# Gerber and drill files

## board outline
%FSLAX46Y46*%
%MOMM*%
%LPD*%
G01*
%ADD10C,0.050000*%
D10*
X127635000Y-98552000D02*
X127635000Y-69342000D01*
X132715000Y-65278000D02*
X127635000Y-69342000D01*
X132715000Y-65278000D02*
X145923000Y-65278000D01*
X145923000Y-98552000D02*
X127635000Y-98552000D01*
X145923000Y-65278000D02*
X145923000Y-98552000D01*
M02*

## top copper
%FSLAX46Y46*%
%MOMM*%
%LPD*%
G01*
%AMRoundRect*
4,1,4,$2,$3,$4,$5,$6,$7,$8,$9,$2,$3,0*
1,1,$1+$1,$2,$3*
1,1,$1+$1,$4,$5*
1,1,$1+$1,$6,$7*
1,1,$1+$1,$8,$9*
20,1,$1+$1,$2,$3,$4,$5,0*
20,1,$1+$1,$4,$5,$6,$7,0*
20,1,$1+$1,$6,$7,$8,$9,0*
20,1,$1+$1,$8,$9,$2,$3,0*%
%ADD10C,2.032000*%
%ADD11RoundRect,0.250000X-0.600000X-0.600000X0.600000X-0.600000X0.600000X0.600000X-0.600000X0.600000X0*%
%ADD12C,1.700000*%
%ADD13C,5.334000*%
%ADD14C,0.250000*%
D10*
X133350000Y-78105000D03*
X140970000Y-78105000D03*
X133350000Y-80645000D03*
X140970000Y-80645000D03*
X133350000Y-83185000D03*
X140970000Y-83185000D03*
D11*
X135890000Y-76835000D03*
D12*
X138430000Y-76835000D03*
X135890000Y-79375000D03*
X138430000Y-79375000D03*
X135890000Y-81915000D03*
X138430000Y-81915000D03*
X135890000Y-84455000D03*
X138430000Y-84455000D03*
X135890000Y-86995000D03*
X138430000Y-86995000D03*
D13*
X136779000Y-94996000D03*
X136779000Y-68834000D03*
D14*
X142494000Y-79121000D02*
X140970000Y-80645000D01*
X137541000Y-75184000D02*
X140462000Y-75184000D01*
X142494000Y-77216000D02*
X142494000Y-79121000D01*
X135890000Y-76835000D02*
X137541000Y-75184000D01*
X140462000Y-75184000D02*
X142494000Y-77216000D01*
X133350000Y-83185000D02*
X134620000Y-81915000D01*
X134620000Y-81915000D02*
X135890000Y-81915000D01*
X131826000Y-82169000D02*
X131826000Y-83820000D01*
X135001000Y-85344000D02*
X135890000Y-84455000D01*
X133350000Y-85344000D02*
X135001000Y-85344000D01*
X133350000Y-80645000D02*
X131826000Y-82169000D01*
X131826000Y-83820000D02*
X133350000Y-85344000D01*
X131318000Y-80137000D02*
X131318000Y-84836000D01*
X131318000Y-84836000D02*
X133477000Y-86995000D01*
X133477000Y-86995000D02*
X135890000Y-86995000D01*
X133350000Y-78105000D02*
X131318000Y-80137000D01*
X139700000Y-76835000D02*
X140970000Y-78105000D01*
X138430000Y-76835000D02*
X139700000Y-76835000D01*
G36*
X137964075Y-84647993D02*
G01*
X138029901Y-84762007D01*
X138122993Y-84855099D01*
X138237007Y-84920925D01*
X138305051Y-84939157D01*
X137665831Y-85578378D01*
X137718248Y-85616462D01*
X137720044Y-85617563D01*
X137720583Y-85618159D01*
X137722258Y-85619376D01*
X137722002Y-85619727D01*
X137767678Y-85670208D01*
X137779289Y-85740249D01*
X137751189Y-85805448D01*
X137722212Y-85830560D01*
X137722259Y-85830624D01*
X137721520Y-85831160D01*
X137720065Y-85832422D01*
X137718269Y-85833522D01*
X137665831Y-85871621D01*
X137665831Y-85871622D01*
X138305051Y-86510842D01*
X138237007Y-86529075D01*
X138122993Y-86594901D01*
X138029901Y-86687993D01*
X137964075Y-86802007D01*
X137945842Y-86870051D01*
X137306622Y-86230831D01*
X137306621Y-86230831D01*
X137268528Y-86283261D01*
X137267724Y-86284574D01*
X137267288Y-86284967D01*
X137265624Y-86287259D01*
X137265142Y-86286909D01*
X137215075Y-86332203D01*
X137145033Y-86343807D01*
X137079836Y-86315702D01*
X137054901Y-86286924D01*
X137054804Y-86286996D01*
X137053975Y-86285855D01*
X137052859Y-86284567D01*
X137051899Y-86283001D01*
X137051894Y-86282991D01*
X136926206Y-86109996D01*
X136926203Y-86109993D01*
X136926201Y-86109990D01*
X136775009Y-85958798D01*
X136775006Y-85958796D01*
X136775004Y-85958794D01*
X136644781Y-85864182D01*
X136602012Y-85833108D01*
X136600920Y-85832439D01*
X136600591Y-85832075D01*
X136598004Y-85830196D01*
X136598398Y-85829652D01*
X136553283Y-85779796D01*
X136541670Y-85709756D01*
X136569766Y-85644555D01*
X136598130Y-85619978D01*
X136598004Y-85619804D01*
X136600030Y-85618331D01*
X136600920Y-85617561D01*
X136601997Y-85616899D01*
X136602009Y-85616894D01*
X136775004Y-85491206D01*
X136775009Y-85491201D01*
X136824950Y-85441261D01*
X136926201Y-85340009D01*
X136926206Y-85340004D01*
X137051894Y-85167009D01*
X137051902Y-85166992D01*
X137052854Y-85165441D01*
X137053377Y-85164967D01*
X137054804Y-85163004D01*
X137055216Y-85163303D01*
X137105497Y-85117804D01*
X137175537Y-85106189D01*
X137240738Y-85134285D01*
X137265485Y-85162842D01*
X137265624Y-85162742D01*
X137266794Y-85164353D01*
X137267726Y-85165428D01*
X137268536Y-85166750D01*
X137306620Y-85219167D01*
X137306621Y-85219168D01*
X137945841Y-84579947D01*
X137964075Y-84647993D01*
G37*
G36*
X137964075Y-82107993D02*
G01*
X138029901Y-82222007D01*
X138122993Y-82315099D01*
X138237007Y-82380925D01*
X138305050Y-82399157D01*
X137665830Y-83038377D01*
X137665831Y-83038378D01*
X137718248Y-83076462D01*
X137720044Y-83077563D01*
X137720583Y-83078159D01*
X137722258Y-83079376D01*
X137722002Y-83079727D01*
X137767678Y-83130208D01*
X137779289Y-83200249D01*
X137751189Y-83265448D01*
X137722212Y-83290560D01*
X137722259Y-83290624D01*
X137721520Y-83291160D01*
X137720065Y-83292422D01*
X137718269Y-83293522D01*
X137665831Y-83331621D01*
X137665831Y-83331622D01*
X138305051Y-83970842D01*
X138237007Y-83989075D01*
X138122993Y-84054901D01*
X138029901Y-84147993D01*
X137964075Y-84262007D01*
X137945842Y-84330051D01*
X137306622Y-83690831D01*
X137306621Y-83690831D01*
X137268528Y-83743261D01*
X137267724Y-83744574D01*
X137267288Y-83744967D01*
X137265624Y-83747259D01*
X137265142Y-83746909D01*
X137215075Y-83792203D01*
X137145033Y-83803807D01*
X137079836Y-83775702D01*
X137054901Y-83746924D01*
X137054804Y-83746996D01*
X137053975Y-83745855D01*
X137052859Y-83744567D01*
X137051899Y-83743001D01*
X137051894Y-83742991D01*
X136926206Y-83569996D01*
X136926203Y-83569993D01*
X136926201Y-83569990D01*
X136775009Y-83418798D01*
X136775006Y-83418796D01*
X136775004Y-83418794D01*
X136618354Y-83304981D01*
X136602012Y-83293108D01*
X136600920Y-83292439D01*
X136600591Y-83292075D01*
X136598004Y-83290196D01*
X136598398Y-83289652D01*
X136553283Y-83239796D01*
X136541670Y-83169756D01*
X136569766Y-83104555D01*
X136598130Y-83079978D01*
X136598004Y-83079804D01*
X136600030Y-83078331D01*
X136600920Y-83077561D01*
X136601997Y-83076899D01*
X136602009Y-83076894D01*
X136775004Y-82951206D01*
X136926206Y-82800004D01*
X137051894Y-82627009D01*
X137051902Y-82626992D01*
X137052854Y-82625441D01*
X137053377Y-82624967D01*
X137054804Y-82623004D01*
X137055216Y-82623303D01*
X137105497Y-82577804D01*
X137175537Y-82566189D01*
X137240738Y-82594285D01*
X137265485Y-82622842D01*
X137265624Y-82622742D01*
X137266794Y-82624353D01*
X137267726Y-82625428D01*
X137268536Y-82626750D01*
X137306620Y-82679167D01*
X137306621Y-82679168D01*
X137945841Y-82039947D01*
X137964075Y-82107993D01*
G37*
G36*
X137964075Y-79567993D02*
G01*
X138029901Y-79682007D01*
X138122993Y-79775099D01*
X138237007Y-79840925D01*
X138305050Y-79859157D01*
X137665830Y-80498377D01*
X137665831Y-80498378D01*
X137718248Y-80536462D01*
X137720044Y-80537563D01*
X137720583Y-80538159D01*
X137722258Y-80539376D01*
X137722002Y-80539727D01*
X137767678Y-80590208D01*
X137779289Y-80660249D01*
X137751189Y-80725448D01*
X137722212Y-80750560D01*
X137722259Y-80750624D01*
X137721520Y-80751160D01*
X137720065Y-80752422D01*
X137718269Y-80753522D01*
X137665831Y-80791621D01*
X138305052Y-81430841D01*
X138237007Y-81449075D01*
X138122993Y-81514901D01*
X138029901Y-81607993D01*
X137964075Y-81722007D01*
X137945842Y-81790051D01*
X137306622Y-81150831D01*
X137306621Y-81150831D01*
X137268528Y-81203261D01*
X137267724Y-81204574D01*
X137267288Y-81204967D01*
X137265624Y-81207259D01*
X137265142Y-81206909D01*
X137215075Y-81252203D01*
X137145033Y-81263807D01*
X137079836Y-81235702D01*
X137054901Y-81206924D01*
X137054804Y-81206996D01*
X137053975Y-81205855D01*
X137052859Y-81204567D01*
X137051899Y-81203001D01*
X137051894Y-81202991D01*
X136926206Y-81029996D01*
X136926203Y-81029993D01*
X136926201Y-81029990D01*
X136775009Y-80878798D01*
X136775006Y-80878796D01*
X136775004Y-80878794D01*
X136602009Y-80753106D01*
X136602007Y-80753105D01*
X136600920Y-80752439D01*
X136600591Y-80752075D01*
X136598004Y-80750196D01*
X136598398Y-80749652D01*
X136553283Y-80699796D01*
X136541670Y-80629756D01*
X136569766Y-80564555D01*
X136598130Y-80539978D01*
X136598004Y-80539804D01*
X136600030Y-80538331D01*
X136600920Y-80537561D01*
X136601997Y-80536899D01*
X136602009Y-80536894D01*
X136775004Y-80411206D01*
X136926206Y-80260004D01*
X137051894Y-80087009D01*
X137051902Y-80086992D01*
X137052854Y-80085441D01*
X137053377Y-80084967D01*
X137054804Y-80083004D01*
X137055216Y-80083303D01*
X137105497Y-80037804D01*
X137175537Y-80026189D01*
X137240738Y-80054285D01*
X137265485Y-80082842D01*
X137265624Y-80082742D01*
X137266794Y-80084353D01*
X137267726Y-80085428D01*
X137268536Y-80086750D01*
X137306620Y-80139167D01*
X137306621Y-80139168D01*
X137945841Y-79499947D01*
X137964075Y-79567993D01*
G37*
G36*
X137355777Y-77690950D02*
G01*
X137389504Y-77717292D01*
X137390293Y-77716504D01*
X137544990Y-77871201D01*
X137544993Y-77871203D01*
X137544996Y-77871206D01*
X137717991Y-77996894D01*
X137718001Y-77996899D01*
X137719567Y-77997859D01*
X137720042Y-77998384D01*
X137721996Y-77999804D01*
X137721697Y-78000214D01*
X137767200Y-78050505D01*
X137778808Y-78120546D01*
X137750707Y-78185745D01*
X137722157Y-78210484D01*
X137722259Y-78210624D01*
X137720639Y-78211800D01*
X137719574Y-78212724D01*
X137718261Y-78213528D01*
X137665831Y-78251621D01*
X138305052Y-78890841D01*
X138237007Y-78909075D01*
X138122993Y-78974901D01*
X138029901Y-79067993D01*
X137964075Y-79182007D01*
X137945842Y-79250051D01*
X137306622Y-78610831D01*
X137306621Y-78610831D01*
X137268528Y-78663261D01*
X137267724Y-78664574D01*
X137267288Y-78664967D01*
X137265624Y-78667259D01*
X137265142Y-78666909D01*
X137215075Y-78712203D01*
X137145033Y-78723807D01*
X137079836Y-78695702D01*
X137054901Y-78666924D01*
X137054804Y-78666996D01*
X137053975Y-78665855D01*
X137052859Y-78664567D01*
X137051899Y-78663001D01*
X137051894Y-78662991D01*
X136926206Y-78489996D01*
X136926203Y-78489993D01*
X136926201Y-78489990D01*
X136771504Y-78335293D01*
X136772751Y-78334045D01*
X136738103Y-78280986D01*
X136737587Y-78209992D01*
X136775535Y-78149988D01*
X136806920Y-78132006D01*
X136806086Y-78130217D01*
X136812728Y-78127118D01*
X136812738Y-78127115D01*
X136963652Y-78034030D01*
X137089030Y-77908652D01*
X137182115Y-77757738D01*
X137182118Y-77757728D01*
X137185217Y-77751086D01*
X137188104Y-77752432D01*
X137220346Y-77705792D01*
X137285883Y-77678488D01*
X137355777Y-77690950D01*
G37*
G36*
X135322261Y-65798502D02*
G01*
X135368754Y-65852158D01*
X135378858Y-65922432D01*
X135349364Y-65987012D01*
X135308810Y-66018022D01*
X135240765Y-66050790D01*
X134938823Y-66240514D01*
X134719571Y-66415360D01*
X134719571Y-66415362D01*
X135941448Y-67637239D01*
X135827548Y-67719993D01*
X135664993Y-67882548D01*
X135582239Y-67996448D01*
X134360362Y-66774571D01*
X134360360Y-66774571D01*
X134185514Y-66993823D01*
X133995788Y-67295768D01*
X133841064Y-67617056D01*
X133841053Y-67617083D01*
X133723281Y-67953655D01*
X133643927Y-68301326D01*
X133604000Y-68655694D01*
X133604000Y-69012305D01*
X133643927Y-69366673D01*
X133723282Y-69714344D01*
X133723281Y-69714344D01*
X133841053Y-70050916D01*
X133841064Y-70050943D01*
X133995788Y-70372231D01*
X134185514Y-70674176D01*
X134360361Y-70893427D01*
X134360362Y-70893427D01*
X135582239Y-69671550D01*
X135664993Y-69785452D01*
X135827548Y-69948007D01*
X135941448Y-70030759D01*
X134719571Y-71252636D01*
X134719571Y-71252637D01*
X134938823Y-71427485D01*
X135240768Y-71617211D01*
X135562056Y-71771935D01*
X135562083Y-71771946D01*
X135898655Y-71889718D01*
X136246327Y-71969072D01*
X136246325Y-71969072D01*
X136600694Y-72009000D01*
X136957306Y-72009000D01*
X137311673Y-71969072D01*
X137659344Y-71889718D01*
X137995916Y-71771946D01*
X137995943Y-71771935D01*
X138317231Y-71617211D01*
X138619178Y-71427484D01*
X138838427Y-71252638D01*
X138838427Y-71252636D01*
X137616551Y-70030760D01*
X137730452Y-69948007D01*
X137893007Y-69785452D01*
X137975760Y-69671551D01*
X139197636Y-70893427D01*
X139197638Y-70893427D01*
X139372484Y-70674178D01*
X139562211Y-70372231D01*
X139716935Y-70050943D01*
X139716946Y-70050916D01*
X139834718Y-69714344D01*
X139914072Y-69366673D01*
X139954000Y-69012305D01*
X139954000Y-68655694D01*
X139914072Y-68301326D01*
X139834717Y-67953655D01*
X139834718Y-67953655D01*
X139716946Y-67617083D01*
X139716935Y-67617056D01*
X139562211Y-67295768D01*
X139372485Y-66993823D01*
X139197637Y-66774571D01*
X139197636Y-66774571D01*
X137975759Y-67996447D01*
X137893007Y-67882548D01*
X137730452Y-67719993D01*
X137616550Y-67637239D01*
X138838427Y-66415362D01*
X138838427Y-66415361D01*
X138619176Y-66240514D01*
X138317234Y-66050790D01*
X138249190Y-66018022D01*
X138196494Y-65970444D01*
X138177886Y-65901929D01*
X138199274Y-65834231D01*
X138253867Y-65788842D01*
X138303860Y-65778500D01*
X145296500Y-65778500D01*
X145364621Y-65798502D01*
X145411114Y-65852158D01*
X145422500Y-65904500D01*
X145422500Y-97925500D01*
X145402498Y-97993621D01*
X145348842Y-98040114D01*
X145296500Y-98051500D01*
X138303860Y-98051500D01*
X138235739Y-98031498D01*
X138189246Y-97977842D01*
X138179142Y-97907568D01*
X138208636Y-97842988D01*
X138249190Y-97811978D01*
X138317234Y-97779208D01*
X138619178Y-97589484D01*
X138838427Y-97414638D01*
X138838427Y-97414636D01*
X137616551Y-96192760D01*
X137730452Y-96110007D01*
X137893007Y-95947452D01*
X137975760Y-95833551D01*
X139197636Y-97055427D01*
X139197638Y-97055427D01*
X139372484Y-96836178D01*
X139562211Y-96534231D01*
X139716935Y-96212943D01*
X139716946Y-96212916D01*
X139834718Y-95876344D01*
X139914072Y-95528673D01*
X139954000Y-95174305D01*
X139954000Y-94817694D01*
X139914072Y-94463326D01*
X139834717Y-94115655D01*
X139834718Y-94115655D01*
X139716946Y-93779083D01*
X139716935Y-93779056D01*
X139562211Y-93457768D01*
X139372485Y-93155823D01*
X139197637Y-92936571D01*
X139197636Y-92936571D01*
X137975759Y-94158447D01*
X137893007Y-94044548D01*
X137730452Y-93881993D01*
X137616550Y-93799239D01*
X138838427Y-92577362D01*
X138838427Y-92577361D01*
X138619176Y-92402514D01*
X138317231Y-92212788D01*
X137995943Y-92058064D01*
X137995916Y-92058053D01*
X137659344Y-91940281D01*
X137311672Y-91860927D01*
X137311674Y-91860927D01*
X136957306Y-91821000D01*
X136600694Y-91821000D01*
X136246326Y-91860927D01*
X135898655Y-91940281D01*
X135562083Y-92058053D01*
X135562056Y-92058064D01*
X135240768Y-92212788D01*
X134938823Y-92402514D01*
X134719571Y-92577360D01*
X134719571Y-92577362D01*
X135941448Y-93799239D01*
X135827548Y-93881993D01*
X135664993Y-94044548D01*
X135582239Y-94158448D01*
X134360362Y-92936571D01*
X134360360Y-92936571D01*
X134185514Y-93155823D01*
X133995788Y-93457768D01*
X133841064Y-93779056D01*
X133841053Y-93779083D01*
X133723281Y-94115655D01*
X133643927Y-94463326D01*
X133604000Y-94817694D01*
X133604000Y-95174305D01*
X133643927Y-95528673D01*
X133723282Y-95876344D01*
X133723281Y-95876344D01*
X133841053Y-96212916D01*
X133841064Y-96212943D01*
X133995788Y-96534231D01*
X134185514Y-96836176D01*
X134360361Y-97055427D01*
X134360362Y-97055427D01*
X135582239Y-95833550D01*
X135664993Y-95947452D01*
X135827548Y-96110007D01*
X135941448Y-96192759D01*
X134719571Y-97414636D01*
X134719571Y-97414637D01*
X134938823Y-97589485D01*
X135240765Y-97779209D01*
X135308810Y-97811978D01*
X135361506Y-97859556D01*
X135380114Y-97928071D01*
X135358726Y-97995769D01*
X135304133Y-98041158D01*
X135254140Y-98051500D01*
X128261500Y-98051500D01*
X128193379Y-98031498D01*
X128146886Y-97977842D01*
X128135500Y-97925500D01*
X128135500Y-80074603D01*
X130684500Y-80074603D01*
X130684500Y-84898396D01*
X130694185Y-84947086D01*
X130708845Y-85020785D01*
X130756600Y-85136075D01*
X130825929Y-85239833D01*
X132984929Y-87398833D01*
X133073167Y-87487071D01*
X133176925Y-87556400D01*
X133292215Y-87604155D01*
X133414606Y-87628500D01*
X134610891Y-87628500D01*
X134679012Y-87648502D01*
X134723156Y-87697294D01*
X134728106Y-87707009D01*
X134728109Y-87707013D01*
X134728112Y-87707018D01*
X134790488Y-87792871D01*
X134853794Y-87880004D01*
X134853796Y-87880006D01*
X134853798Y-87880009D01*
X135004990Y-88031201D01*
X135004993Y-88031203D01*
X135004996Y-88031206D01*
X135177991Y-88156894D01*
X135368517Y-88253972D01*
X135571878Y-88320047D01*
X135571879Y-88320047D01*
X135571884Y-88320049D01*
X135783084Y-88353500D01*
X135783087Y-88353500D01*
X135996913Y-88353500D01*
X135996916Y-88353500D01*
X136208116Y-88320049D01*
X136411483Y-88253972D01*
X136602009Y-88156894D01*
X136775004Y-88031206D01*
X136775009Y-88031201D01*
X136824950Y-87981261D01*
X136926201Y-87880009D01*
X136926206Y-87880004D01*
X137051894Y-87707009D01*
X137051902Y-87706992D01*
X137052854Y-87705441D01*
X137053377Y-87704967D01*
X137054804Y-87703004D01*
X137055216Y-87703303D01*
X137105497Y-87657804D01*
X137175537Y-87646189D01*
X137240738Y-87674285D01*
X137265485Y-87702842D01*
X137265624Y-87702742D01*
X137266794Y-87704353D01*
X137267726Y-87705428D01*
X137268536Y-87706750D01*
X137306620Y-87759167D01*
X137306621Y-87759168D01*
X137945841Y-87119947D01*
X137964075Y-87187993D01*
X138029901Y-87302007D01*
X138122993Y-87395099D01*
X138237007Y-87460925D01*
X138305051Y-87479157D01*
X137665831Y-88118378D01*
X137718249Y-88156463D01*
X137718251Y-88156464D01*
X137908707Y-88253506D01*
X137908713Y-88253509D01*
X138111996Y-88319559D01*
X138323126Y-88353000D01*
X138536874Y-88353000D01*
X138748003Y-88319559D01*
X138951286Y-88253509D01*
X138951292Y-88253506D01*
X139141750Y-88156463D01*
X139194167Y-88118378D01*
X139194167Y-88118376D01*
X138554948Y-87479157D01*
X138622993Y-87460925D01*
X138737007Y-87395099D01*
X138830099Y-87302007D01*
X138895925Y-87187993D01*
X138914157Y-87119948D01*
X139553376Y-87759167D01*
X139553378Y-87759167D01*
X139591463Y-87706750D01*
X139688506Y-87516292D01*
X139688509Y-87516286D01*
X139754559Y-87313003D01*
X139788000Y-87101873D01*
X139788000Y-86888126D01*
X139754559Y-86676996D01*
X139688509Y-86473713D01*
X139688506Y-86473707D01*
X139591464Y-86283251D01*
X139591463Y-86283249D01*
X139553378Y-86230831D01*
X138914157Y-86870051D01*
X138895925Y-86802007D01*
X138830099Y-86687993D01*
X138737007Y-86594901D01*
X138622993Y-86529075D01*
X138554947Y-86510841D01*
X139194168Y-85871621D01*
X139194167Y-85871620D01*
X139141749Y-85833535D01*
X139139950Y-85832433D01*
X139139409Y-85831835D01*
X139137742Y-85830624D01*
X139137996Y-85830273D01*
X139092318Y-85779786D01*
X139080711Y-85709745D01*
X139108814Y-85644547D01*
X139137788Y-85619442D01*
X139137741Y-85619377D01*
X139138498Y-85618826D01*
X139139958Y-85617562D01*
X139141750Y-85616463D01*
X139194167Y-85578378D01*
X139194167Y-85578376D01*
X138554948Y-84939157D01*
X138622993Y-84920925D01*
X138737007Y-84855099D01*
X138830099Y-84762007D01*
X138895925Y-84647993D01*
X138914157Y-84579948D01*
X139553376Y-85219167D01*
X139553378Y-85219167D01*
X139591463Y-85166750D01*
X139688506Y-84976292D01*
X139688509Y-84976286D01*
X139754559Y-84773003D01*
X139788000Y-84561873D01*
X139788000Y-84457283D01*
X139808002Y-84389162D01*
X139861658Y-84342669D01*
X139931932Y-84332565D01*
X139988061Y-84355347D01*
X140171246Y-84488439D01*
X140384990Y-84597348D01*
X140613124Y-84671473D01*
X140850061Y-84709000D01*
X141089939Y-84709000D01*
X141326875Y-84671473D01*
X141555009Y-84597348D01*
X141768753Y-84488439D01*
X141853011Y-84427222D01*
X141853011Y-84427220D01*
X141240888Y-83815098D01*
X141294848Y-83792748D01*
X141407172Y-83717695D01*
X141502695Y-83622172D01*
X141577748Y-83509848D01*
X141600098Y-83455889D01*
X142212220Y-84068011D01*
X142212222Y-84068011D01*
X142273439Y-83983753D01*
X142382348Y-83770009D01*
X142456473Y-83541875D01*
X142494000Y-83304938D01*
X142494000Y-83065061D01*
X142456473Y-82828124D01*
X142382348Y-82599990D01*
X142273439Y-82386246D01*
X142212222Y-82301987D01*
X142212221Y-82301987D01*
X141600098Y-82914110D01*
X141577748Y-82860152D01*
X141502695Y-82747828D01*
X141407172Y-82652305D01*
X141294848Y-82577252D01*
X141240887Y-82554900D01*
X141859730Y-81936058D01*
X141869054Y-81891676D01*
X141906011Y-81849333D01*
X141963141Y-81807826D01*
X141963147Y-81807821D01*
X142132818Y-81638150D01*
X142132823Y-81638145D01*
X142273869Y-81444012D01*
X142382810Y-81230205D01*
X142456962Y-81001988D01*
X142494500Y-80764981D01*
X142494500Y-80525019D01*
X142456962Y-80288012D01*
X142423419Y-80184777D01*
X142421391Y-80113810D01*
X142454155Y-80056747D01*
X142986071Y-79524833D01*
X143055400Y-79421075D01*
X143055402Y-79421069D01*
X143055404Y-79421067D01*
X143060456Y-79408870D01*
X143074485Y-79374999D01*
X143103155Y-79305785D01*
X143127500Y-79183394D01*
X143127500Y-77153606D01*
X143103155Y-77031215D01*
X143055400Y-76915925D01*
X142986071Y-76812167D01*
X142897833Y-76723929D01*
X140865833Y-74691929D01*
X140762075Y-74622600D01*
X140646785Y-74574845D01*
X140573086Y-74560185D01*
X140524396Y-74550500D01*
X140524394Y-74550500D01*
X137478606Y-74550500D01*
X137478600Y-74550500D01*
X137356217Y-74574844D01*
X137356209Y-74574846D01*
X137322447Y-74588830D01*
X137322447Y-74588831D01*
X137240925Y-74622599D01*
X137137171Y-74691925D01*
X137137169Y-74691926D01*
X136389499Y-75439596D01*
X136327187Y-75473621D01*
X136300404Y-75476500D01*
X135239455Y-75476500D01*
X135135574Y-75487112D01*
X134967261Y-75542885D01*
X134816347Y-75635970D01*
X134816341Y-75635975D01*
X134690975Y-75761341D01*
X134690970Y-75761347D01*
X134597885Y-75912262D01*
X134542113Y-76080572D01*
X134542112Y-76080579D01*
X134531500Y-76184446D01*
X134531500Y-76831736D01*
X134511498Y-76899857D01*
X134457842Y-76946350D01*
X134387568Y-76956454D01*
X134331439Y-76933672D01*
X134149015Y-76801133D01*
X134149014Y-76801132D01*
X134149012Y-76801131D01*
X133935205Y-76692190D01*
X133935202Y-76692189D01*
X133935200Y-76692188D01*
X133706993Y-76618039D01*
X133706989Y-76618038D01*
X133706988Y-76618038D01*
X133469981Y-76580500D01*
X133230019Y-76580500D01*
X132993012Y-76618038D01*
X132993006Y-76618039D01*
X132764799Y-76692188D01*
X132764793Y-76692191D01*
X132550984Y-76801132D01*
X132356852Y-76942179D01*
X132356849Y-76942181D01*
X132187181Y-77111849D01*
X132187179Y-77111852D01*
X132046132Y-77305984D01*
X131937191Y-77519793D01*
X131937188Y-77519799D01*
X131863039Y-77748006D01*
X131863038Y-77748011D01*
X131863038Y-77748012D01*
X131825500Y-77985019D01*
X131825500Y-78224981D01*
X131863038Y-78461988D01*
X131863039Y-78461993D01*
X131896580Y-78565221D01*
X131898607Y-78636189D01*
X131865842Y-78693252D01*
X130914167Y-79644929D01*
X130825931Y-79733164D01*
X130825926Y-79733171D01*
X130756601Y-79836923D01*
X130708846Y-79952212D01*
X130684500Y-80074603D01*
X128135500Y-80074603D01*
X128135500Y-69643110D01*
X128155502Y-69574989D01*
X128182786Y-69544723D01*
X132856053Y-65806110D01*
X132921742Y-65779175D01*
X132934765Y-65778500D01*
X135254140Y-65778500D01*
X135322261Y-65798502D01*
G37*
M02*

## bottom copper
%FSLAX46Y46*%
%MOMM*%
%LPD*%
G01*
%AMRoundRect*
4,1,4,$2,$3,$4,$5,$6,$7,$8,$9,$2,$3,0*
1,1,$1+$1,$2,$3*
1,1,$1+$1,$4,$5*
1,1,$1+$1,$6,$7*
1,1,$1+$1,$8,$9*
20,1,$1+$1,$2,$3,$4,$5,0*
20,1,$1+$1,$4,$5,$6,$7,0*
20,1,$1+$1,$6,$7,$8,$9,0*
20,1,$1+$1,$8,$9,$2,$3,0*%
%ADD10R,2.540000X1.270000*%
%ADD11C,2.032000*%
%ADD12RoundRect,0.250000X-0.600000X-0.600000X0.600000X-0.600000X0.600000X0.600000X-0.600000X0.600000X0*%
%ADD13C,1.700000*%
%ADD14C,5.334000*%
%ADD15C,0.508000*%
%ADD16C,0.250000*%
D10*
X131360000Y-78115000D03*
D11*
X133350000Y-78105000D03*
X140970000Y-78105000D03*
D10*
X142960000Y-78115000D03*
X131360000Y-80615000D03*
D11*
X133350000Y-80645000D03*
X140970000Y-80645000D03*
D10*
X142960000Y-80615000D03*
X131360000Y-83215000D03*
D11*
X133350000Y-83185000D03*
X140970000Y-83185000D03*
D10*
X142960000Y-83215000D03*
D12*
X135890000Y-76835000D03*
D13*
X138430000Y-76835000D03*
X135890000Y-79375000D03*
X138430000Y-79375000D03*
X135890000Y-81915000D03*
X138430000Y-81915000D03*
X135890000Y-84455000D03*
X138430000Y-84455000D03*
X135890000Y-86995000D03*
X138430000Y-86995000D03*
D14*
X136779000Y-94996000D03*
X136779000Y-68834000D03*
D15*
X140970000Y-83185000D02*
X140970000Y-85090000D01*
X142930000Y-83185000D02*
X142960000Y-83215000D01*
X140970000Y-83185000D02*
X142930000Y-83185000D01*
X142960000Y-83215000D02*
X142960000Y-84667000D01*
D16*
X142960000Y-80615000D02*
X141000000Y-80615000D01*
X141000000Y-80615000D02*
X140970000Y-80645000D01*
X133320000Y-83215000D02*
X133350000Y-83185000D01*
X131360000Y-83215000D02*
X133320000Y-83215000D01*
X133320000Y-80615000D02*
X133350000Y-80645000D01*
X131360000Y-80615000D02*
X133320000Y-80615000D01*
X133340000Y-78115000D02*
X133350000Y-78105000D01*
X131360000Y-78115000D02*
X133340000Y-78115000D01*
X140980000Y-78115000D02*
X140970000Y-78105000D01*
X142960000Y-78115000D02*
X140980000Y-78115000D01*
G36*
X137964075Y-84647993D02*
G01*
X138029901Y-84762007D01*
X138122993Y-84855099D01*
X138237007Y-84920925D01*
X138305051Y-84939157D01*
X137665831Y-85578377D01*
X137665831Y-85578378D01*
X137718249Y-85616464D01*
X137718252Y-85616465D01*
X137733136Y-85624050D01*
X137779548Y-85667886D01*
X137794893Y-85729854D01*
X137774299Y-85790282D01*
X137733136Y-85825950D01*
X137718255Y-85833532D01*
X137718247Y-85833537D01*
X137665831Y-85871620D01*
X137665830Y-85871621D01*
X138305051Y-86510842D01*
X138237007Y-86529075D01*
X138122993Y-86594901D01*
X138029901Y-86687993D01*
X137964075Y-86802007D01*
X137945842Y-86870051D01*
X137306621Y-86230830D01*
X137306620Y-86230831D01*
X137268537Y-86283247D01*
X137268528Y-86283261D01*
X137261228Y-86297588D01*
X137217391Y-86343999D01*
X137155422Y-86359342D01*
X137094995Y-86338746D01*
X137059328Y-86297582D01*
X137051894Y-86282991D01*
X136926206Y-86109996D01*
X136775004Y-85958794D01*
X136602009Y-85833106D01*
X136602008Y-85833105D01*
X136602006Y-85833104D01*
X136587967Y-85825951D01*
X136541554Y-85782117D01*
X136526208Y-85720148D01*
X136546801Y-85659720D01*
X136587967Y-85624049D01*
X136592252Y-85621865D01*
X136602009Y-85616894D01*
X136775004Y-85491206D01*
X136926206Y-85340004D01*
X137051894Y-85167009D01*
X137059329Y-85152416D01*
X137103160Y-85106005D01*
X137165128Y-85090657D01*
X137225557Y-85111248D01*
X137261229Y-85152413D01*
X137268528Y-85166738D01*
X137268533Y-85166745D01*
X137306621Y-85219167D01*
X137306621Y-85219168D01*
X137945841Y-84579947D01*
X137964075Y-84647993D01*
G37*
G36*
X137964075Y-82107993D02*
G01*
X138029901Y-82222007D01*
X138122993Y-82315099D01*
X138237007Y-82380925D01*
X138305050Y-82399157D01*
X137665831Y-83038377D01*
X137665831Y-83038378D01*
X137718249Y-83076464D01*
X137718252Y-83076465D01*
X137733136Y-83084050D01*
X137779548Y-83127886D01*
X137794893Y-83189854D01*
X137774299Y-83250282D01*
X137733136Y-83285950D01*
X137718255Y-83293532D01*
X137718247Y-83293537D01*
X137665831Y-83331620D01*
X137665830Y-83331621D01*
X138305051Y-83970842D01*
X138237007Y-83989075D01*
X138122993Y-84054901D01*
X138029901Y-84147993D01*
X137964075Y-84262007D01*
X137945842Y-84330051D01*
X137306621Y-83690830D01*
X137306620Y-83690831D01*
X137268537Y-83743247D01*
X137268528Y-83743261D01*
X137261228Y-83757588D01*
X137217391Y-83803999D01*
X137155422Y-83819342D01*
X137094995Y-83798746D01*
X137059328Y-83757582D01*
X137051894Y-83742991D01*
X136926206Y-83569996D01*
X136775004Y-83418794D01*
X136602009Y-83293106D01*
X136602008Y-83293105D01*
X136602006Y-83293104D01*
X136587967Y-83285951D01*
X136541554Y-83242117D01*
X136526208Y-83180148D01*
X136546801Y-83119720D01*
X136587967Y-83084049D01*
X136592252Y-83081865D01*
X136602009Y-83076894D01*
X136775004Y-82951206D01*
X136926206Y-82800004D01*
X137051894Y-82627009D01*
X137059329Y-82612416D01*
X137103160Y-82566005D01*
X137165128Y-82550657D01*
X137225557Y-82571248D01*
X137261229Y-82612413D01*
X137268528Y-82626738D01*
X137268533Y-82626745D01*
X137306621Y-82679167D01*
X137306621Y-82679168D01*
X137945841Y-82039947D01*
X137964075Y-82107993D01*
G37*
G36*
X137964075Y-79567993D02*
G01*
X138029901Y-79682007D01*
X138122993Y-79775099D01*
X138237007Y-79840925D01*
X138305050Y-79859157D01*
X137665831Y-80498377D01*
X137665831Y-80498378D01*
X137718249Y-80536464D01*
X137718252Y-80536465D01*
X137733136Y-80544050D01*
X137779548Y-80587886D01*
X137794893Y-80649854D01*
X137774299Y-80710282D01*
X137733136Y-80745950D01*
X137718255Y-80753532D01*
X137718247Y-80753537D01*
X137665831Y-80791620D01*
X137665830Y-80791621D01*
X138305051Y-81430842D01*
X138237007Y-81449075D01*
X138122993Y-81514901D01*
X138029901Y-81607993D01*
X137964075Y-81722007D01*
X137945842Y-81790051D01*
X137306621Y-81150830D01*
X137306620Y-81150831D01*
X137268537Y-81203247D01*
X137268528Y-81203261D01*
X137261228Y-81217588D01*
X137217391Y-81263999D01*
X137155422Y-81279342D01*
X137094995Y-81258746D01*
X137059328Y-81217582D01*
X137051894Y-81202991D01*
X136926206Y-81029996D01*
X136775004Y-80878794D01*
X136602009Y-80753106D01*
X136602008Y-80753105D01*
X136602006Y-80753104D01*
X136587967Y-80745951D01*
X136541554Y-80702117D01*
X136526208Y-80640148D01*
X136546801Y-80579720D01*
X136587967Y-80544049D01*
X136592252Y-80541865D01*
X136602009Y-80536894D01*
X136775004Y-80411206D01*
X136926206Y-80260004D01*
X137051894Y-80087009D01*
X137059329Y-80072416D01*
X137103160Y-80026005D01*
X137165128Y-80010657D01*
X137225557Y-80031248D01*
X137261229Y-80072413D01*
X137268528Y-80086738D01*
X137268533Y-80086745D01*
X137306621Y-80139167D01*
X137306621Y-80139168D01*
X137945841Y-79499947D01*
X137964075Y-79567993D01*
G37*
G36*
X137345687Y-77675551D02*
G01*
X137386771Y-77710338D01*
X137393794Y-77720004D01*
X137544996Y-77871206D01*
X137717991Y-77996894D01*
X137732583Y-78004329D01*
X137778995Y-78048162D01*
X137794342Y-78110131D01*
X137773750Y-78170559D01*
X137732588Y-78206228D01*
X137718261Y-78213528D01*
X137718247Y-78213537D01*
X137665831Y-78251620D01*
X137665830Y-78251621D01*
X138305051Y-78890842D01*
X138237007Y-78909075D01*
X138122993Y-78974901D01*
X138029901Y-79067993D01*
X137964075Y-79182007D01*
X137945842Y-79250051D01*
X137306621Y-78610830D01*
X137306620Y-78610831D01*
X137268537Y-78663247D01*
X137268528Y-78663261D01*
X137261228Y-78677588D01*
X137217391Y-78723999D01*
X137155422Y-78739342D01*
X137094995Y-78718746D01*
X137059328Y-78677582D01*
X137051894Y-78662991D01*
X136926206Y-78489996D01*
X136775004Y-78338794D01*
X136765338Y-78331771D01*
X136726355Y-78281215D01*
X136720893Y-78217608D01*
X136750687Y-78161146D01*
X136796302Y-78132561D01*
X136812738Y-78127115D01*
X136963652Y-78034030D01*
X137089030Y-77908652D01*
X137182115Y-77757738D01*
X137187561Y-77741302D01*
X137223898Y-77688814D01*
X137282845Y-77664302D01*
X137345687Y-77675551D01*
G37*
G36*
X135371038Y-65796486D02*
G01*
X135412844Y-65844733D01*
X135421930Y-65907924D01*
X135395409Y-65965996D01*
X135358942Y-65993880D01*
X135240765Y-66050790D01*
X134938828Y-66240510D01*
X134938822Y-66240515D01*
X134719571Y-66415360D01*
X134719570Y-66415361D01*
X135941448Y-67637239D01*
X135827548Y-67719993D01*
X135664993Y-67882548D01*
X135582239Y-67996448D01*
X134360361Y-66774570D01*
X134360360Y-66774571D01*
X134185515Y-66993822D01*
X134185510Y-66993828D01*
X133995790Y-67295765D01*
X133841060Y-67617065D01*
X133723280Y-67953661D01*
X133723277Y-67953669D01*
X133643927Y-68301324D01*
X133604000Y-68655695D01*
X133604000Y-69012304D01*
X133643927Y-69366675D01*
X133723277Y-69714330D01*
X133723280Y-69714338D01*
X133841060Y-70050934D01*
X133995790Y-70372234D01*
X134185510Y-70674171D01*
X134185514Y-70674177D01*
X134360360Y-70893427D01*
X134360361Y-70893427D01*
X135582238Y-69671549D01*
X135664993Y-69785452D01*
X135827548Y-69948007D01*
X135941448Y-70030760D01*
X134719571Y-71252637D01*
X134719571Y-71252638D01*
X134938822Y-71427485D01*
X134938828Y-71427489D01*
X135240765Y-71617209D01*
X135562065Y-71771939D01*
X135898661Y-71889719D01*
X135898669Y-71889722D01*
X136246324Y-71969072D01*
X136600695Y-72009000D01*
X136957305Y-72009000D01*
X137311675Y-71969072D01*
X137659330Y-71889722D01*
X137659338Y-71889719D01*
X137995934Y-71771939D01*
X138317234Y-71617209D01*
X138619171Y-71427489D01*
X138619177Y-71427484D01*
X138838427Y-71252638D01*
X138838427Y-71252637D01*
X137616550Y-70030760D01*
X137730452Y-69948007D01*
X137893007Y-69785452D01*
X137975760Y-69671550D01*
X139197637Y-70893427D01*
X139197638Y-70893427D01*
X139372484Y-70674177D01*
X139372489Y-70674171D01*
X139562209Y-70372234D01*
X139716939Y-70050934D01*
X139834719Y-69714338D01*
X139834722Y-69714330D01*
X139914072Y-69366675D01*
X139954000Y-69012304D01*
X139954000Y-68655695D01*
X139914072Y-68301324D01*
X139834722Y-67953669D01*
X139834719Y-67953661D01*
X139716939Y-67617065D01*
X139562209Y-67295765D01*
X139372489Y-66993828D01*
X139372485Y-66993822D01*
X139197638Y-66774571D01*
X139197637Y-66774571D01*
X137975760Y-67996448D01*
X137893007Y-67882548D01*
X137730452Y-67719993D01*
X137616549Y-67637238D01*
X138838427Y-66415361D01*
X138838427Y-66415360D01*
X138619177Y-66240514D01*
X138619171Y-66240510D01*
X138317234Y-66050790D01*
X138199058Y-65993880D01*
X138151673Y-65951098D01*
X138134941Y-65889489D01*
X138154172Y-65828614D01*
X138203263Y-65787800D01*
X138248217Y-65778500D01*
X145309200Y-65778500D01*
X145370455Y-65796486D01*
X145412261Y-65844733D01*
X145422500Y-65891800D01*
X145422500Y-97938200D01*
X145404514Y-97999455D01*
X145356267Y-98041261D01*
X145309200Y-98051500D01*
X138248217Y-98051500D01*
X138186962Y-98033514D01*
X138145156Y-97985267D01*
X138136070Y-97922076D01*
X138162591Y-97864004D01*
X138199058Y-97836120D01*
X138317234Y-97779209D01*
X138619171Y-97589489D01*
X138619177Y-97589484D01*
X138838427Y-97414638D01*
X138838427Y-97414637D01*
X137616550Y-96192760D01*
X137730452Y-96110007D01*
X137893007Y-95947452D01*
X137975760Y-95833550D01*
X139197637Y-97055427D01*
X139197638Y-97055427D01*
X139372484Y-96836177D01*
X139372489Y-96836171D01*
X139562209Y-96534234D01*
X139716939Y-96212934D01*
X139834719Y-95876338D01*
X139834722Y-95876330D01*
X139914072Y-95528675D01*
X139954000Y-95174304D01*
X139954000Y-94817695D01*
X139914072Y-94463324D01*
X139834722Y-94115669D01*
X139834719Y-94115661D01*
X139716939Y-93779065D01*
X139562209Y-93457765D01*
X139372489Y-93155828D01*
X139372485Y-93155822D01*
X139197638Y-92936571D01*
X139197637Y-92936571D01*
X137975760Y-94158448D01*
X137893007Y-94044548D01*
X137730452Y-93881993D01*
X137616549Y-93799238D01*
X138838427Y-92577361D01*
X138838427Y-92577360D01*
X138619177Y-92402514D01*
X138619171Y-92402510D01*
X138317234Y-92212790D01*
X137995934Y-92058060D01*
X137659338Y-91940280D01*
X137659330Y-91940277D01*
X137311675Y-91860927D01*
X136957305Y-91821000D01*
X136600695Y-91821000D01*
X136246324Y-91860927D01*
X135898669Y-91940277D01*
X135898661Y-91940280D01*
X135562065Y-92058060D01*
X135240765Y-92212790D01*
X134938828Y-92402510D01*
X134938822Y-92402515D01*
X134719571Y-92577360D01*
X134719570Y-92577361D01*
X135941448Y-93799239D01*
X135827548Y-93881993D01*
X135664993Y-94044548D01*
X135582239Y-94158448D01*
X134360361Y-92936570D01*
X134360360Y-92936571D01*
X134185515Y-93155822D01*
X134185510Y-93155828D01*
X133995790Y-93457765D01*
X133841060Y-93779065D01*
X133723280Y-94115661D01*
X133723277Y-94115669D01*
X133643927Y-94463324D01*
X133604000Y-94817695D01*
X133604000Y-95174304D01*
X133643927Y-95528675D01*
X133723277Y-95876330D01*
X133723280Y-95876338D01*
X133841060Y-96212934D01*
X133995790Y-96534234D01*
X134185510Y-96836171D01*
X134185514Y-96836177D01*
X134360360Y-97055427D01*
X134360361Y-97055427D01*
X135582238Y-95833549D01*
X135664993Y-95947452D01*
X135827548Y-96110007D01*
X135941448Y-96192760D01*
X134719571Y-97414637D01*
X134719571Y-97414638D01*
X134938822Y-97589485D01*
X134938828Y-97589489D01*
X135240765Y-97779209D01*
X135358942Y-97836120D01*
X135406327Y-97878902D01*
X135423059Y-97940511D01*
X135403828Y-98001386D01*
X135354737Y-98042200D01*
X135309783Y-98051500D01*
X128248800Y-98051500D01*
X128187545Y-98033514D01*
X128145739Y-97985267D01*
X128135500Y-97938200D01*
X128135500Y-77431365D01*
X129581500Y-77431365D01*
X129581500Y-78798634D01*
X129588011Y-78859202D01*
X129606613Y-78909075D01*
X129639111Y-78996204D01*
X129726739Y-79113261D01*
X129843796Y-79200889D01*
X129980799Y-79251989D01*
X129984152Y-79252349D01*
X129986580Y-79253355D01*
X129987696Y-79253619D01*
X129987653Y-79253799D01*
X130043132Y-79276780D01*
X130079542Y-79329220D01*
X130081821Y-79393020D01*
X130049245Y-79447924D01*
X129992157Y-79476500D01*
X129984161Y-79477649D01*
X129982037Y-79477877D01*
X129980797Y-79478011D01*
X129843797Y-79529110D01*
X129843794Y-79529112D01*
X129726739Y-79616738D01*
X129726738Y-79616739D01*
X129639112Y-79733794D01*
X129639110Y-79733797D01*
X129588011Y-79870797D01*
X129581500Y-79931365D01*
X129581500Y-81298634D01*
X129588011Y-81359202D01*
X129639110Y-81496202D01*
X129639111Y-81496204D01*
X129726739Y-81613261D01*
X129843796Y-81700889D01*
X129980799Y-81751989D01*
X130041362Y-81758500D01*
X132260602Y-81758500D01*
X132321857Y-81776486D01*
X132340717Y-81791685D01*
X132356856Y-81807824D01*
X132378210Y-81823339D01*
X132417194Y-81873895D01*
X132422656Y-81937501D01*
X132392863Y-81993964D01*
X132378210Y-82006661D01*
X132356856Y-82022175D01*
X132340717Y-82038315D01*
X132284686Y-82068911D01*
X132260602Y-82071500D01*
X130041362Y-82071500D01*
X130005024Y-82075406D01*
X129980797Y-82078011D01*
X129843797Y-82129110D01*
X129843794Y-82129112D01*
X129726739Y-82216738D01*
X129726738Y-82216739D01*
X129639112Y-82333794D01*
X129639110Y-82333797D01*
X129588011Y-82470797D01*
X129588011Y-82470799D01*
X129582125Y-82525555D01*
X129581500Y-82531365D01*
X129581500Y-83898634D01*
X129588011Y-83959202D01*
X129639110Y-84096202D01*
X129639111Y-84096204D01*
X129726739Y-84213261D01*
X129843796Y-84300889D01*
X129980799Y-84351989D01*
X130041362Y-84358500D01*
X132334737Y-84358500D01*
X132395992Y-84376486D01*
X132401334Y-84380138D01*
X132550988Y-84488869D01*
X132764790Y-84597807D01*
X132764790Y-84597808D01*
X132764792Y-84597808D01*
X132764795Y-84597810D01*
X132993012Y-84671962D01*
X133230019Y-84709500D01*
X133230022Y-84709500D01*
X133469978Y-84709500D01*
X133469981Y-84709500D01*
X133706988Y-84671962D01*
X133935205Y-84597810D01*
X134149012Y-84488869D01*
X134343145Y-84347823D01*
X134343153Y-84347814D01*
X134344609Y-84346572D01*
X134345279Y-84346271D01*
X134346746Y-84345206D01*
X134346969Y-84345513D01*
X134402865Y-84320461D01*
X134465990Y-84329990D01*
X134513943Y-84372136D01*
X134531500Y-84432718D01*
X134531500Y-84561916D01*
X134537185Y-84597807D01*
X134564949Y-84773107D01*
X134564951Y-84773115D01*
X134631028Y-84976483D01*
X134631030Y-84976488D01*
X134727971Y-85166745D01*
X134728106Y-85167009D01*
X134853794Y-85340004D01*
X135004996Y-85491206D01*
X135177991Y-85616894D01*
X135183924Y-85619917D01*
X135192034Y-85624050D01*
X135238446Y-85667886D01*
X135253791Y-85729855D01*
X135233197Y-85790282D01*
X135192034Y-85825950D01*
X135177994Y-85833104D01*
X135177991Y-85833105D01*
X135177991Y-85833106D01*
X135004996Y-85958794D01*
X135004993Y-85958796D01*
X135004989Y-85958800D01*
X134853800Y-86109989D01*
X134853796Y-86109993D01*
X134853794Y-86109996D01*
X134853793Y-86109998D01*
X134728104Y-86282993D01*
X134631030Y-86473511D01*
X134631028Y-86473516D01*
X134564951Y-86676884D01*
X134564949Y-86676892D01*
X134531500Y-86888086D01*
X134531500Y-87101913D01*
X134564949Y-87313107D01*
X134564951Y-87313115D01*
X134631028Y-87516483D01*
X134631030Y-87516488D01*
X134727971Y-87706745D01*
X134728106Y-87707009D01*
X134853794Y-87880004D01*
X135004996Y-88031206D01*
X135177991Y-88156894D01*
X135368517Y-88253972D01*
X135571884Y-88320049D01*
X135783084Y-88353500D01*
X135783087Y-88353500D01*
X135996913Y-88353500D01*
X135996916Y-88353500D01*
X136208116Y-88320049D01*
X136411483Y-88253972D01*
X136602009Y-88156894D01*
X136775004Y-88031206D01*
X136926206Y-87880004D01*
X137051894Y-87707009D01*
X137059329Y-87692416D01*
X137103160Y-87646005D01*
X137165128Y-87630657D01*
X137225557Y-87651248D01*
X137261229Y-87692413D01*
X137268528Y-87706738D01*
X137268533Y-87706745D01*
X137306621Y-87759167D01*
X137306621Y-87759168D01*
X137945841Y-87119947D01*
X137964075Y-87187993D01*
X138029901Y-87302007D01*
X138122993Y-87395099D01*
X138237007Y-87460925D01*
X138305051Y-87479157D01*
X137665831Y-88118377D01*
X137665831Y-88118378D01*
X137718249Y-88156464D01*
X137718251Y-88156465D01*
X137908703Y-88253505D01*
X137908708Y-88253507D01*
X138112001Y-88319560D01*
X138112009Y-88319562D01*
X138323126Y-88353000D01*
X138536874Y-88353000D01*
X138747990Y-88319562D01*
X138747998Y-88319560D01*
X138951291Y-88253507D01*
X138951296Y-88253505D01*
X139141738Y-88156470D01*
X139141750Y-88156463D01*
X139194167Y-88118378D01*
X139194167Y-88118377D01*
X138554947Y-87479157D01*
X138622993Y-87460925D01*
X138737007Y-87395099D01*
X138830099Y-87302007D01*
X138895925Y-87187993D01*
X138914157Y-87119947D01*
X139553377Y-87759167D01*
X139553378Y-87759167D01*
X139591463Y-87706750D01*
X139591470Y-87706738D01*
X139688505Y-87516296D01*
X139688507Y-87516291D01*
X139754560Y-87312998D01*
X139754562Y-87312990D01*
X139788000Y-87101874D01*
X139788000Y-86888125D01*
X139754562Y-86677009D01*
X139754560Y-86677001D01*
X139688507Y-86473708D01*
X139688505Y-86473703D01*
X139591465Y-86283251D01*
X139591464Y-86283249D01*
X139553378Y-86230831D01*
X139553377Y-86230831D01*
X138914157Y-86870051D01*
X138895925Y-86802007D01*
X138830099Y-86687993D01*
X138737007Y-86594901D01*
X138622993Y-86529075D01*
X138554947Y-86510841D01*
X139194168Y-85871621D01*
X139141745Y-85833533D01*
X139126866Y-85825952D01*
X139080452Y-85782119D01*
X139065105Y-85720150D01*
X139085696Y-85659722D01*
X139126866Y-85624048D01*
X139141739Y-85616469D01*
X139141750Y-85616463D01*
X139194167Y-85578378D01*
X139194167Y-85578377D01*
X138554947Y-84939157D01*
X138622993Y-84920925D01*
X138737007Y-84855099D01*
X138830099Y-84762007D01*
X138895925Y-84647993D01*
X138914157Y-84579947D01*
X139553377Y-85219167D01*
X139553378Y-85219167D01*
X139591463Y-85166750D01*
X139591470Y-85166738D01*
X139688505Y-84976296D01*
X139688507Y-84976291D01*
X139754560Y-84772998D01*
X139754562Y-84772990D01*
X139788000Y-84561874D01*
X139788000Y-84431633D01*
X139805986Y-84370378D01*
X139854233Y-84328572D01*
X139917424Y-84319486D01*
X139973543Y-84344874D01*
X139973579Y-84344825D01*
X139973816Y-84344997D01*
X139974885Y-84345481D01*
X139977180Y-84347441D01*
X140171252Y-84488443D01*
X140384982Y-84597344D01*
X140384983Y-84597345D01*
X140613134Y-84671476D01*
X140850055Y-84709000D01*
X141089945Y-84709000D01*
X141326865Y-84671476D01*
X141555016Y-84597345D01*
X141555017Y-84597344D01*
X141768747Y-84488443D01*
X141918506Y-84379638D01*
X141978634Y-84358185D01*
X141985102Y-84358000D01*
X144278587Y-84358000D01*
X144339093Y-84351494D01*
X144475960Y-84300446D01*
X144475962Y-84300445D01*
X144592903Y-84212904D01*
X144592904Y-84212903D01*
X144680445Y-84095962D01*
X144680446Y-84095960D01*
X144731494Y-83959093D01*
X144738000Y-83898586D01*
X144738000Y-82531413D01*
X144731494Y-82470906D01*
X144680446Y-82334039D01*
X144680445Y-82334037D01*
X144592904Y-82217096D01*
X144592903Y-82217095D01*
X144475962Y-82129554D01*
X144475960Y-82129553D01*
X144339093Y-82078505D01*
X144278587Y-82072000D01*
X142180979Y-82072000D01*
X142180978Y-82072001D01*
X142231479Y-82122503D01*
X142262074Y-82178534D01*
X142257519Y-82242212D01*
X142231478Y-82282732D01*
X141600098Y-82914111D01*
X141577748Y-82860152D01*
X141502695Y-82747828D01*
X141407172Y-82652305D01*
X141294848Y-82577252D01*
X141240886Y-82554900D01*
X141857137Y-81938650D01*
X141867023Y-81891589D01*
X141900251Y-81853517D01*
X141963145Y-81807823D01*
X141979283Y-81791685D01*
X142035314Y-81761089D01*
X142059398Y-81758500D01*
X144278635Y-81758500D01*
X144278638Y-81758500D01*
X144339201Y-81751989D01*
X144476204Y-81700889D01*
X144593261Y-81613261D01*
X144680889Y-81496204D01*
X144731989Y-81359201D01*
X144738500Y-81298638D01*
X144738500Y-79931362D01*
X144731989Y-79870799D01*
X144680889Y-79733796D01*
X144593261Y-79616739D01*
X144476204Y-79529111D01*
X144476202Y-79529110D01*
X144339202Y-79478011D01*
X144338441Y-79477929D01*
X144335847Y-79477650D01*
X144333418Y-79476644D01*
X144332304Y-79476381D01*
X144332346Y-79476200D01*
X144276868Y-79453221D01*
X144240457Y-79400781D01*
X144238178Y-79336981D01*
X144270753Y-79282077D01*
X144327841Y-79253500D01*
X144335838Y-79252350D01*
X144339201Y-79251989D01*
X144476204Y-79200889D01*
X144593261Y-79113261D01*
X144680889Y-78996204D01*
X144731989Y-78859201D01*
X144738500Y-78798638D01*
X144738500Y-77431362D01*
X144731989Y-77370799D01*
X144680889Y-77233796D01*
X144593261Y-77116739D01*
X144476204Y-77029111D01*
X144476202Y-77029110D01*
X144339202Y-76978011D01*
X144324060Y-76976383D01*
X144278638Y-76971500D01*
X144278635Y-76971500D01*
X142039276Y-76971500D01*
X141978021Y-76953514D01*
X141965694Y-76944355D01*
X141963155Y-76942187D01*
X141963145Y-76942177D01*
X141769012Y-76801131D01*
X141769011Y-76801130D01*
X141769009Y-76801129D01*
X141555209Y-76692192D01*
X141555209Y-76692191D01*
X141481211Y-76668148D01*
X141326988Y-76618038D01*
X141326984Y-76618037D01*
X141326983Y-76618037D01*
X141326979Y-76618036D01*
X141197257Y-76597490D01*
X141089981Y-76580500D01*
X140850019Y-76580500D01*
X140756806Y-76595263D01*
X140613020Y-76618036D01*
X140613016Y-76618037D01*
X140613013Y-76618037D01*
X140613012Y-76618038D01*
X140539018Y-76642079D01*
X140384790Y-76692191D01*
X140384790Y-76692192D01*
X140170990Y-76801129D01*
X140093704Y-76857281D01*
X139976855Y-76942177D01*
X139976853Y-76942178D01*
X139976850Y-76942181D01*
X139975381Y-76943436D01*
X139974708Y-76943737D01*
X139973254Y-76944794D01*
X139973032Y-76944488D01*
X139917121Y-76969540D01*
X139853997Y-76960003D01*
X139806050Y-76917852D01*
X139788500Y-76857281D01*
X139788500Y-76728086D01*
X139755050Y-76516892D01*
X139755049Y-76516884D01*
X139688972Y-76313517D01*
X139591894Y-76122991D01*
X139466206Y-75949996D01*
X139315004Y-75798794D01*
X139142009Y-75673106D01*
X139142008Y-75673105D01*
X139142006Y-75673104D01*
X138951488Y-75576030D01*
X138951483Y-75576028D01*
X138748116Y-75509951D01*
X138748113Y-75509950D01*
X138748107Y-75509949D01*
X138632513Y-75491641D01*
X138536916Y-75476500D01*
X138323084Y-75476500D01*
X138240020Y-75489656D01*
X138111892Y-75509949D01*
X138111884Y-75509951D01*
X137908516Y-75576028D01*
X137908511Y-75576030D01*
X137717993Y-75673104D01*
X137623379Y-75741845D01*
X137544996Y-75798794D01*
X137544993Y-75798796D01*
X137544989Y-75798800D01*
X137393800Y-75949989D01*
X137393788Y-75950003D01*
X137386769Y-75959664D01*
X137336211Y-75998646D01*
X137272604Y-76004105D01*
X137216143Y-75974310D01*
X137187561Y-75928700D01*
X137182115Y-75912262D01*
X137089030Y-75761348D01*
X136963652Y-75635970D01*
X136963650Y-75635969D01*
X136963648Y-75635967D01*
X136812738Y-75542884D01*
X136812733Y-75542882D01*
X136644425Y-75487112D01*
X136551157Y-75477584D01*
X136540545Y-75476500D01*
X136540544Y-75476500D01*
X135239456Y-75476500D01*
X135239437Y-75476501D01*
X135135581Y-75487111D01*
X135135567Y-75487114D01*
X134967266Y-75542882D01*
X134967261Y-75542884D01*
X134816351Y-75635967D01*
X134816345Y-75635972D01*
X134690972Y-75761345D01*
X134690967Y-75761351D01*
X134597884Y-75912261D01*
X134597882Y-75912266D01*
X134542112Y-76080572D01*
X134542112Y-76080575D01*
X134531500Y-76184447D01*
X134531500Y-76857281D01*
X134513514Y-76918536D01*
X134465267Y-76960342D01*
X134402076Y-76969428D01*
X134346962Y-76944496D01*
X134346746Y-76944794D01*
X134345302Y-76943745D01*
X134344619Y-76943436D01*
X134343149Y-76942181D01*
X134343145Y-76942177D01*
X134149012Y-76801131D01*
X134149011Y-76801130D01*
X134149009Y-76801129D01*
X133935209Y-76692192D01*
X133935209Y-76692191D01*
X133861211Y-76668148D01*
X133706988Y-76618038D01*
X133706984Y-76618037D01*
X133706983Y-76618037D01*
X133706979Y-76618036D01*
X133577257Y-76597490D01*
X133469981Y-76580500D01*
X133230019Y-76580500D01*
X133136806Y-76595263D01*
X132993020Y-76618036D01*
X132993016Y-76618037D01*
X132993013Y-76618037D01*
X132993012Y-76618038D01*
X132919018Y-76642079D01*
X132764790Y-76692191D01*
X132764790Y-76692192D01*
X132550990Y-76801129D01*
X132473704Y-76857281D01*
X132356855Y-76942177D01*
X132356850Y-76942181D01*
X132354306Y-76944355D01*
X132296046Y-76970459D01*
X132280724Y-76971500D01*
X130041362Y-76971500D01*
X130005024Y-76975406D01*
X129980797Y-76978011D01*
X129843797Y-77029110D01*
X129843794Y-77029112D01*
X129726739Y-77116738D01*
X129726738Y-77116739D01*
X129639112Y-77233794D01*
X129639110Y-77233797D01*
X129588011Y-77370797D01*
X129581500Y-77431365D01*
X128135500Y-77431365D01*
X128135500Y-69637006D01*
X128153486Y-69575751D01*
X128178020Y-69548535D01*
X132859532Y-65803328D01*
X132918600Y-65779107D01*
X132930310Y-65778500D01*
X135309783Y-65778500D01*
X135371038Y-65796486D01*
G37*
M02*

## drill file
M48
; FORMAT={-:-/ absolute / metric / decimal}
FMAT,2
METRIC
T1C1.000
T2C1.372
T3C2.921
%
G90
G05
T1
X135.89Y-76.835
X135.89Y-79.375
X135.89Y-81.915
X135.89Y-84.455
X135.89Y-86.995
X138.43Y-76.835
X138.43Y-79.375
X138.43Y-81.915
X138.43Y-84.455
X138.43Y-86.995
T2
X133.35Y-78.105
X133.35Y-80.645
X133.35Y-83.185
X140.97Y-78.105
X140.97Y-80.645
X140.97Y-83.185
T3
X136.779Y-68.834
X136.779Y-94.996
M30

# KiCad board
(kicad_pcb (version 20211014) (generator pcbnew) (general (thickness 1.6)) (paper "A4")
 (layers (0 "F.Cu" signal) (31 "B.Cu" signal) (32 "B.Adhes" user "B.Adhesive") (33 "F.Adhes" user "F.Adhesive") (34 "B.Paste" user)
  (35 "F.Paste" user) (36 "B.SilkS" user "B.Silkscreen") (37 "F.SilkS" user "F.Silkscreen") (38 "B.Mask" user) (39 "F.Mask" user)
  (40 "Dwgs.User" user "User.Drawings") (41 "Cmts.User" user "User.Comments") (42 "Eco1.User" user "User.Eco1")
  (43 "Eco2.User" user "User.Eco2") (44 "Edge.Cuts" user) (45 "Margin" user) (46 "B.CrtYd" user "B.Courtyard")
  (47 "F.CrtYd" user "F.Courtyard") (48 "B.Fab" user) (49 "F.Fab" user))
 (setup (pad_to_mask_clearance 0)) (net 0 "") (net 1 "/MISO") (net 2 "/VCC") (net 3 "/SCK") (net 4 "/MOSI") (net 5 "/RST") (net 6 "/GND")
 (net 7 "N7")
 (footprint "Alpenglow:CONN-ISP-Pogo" (layer "F.Cu") (at 137.16 81.915)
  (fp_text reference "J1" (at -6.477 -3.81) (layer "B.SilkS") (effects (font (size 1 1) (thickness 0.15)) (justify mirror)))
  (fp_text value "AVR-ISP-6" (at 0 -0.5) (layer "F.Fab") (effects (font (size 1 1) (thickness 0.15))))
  (pad "1" smd rect locked (at -5.8 -3.8) (size 2.54 1.27) (layers "B.Cu" "B.Paste" "B.Mask") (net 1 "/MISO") (zone_connect 0))
  (pad "1" thru_hole circle locked (at -3.81 -3.81) (size 2.032 2.032) (drill 1.3716) (layers *.Cu *.Mask) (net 1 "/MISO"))
  (pad "2" thru_hole circle locked (at 3.81 -3.81) (size 2.032 2.032) (drill 1.3716) (layers *.Cu *.Mask) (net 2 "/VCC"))
  (pad "2" smd rect locked (at 5.8 -3.8) (size 2.54 1.27) (layers "B.Cu" "B.Paste" "B.Mask") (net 2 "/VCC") (zone_connect 0))
  (pad "3" smd rect locked (at -5.8 -1.3) (size 2.54 1.27) (layers "B.Cu" "B.Paste" "B.Mask") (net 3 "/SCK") (zone_connect 0))
  (pad "3" thru_hole circle locked (at -3.81 -1.27) (size 2.032 2.032) (drill 1.3716) (layers *.Cu *.Mask) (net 3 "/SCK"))
  (pad "4" thru_hole circle locked (at 3.81 -1.27) (size 2.032 2.032) (drill 1.3716) (layers *.Cu *.Mask) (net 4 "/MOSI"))
  (pad "4" smd rect locked (at 5.8 -1.3) (size 2.54 1.27) (layers "B.Cu" "B.Paste" "B.Mask") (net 4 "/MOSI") (zone_connect 0))
  (pad "5" smd rect locked (at -5.8 1.3) (size 2.54 1.27) (layers "B.Cu" "B.Paste" "B.Mask") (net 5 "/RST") (zone_connect 0))
  (pad "5" thru_hole circle locked (at -3.81 1.27) (size 2.032 2.032) (drill 1.3716) (layers *.Cu *.Mask) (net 5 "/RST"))
  (pad "6" thru_hole circle locked (at 3.81 1.27) (size 2.032 2.032) (drill 1.3716) (layers *.Cu *.Mask) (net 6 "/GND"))
  (pad "6" smd rect locked (at 5.8 1.3) (size 2.54 1.27) (layers "B.Cu" "B.Paste" "B.Mask") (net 6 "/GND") (zone_connect 0)))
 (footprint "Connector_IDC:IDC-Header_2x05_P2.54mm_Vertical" (layer "F.Cu") (at 135.89 76.835)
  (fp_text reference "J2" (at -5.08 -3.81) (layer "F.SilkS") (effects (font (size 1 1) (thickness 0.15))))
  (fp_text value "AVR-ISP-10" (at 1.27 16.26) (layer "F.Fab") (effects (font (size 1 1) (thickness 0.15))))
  (pad "1" thru_hole roundrect locked (at 0 0) (size 1.7 1.7) (drill 1) (layers *.Cu *.Mask) (roundrect_rratio 0.1470588235) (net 4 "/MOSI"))
  (pad "2" thru_hole circle locked (at 2.54 0) (size 1.7 1.7) (drill 1) (layers *.Cu *.Mask) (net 2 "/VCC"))
  (pad "3" thru_hole circle locked (at 0 2.54) (size 1.7 1.7) (drill 1) (layers *.Cu *.Mask) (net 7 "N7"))
  (pad "4" thru_hole circle locked (at 2.54 2.54) (size 1.7 1.7) (drill 1) (layers *.Cu *.Mask) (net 6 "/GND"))
  (pad "5" thru_hole circle locked (at 0 5.08) (size 1.7 1.7) (drill 1) (layers *.Cu *.Mask) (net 5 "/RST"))
  (pad "6" thru_hole circle locked (at 2.54 5.08) (size 1.7 1.7) (drill 1) (layers *.Cu *.Mask) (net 6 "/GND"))
  (pad "7" thru_hole circle locked (at 0 7.62) (size 1.7 1.7) (drill 1) (layers *.Cu *.Mask) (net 3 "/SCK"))
  (pad "8" thru_hole circle locked (at 2.54 7.62) (size 1.7 1.7) (drill 1) (layers *.Cu *.Mask) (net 6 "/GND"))
  (pad "9" thru_hole circle locked (at 0 10.16) (size 1.7 1.7) (drill 1) (layers *.Cu *.Mask) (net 1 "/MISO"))
  (pad "10" thru_hole circle locked (at 2.54 10.16) (size 1.7 1.7) (drill 1) (layers *.Cu *.Mask) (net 6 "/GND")))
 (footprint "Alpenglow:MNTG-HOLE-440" (layer "F.Cu") (at 136.779 93.726)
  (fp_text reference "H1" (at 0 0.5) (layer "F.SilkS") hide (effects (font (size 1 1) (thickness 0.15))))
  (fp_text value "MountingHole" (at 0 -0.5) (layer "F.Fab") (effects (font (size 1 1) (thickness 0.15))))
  (pad "1" thru_hole circle locked (at 0 1.27) (size 5.334 5.334) (drill 2.921) (layers *.Cu *.Mask) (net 6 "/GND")))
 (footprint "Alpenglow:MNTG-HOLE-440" (layer "F.Cu") (at 136.779 67.564)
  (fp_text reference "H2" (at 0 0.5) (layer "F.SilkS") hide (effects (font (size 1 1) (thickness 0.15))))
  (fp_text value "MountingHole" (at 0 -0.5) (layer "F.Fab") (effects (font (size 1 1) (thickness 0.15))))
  (pad "1" thru_hole circle locked (at 0 1.27) (size 5.334 5.334) (drill 2.921) (layers *.Cu *.Mask) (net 6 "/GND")))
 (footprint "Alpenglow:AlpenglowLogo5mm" (layer "B.Cu") (at 142.24 90.17 180)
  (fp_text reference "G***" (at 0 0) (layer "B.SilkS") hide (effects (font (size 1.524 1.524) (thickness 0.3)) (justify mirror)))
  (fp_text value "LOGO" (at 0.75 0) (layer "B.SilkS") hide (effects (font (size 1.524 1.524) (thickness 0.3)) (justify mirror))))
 (gr_line (start 127.635 98.552) (end 127.635 69.342) (layer "Edge.Cuts") (width 0.05))
 (gr_line (start 132.715 65.278) (end 127.635 69.342) (layer "Edge.Cuts") (width 0.05))
 (gr_line (start 132.715 65.278) (end 145.923 65.278) (layer "Edge.Cuts") (width 0.05))
 (gr_line (start 145.923 98.552) (end 127.635 98.552) (layer "Edge.Cuts") (width 0.05))
 (gr_line (start 145.923 65.278) (end 145.923 98.552) (layer "Edge.Cuts") (width 0.05))
 (segment (start 140.97 83.185) (end 140.97 85.09) (width 0.508) (layer "B.Cu") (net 6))
 (segment (start 142.93 83.185) (end 142.96 83.215) (width 0.508) (layer "B.Cu") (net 6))
 (segment (start 140.97 83.185) (end 142.93 83.185) (width 0.508) (layer "B.Cu") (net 6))
 (segment (start 142.96 83.215) (end 142.96 84.667) (width 0.508) (layer "B.Cu") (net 6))
 (segment (start 142.494 79.121) (end 140.97 80.645) (width 0.25) (layer "F.Cu") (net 4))
 (segment (start 137.541 75.184) (end 140.462 75.184) (width 0.25) (layer "F.Cu") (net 4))
 (segment (start 142.494 77.216) (end 142.494 79.121) (width 0.25) (layer "F.Cu") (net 4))
 (segment (start 135.89 76.835) (end 137.541 75.184) (width 0.25) (layer "F.Cu") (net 4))
 (segment (start 140.462 75.184) (end 142.494 77.216) (width 0.25) (layer "F.Cu") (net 4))
 (segment (start 142.96 80.615) (end 141 80.615) (width 0.25) (layer "B.Cu") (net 4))
 (segment (start 141 80.615) (end 140.97 80.645) (width 0.25) (layer "B.Cu") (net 4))
 (segment (start 133.35 83.185) (end 134.62 81.915) (width 0.25) (layer "F.Cu") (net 5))
 (segment (start 134.62 81.915) (end 135.89 81.915) (width 0.25) (layer "F.Cu") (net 5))
 (segment (start 133.32 83.215) (end 133.35 83.185) (width 0.25) (layer "B.Cu") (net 5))
 (segment (start 131.36 83.215) (end 133.32 83.215) (width 0.25) (layer "B.Cu") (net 5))
 (segment (start 131.826 82.169) (end 131.826 83.82) (width 0.25) (layer "F.Cu") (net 3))
 (segment (start 135.001 85.344) (end 135.89 84.455) (width 0.25) (layer "F.Cu") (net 3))
 (segment (start 133.35 85.344) (end 135.001 85.344) (width 0.25) (layer "F.Cu") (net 3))
 (segment (start 133.35 80.645) (end 131.826 82.169) (width 0.25) (layer "F.Cu") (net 3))
 (segment (start 131.826 83.82) (end 133.35 85.344) (width 0.25) (layer "F.Cu") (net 3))
 (segment (start 133.32 80.615) (end 133.35 80.645) (width 0.25) (layer "B.Cu") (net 3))
 (segment (start 131.36 80.615) (end 133.32 80.615) (width 0.25) (layer "B.Cu") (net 3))
 (segment (start 131.318 80.137) (end 131.318 84.836) (width 0.25) (layer "F.Cu") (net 1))
 (segment (start 131.318 84.836) (end 133.477 86.995) (width 0.25) (layer "F.Cu") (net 1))
 (segment (start 133.477 86.995) (end 135.89 86.995) (width 0.25) (layer "F.Cu") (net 1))
 (segment (start 133.35 78.105) (end 131.318 80.137) (width 0.25) (layer "F.Cu") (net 1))
 (segment (start 133.34 78.115) (end 133.35 78.105) (width 0.25) (layer "B.Cu") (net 1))
 (segment (start 131.36 78.115) (end 133.34 78.115) (width 0.25) (layer "B.Cu") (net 1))
 (segment (start 139.7 76.835) (end 140.97 78.105) (width 0.25) (layer "F.Cu") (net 2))
 (segment (start 138.43 76.835) (end 139.7 76.835) (width 0.25) (layer "F.Cu") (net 2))
 (segment (start 140.98 78.115) (end 140.97 78.105) (width 0.25) (layer "B.Cu") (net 2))
 (segment (start 142.96 78.115) (end 140.98 78.115) (width 0.25) (layer "B.Cu") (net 2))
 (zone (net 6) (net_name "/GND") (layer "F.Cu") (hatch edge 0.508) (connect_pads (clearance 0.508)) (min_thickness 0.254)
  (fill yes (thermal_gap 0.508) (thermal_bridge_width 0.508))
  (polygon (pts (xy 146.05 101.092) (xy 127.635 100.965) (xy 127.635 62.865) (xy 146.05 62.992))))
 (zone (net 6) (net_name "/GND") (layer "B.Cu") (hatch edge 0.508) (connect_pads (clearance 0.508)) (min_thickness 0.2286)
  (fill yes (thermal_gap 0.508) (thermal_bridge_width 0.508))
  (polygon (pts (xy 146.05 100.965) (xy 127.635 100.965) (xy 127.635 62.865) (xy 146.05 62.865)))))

